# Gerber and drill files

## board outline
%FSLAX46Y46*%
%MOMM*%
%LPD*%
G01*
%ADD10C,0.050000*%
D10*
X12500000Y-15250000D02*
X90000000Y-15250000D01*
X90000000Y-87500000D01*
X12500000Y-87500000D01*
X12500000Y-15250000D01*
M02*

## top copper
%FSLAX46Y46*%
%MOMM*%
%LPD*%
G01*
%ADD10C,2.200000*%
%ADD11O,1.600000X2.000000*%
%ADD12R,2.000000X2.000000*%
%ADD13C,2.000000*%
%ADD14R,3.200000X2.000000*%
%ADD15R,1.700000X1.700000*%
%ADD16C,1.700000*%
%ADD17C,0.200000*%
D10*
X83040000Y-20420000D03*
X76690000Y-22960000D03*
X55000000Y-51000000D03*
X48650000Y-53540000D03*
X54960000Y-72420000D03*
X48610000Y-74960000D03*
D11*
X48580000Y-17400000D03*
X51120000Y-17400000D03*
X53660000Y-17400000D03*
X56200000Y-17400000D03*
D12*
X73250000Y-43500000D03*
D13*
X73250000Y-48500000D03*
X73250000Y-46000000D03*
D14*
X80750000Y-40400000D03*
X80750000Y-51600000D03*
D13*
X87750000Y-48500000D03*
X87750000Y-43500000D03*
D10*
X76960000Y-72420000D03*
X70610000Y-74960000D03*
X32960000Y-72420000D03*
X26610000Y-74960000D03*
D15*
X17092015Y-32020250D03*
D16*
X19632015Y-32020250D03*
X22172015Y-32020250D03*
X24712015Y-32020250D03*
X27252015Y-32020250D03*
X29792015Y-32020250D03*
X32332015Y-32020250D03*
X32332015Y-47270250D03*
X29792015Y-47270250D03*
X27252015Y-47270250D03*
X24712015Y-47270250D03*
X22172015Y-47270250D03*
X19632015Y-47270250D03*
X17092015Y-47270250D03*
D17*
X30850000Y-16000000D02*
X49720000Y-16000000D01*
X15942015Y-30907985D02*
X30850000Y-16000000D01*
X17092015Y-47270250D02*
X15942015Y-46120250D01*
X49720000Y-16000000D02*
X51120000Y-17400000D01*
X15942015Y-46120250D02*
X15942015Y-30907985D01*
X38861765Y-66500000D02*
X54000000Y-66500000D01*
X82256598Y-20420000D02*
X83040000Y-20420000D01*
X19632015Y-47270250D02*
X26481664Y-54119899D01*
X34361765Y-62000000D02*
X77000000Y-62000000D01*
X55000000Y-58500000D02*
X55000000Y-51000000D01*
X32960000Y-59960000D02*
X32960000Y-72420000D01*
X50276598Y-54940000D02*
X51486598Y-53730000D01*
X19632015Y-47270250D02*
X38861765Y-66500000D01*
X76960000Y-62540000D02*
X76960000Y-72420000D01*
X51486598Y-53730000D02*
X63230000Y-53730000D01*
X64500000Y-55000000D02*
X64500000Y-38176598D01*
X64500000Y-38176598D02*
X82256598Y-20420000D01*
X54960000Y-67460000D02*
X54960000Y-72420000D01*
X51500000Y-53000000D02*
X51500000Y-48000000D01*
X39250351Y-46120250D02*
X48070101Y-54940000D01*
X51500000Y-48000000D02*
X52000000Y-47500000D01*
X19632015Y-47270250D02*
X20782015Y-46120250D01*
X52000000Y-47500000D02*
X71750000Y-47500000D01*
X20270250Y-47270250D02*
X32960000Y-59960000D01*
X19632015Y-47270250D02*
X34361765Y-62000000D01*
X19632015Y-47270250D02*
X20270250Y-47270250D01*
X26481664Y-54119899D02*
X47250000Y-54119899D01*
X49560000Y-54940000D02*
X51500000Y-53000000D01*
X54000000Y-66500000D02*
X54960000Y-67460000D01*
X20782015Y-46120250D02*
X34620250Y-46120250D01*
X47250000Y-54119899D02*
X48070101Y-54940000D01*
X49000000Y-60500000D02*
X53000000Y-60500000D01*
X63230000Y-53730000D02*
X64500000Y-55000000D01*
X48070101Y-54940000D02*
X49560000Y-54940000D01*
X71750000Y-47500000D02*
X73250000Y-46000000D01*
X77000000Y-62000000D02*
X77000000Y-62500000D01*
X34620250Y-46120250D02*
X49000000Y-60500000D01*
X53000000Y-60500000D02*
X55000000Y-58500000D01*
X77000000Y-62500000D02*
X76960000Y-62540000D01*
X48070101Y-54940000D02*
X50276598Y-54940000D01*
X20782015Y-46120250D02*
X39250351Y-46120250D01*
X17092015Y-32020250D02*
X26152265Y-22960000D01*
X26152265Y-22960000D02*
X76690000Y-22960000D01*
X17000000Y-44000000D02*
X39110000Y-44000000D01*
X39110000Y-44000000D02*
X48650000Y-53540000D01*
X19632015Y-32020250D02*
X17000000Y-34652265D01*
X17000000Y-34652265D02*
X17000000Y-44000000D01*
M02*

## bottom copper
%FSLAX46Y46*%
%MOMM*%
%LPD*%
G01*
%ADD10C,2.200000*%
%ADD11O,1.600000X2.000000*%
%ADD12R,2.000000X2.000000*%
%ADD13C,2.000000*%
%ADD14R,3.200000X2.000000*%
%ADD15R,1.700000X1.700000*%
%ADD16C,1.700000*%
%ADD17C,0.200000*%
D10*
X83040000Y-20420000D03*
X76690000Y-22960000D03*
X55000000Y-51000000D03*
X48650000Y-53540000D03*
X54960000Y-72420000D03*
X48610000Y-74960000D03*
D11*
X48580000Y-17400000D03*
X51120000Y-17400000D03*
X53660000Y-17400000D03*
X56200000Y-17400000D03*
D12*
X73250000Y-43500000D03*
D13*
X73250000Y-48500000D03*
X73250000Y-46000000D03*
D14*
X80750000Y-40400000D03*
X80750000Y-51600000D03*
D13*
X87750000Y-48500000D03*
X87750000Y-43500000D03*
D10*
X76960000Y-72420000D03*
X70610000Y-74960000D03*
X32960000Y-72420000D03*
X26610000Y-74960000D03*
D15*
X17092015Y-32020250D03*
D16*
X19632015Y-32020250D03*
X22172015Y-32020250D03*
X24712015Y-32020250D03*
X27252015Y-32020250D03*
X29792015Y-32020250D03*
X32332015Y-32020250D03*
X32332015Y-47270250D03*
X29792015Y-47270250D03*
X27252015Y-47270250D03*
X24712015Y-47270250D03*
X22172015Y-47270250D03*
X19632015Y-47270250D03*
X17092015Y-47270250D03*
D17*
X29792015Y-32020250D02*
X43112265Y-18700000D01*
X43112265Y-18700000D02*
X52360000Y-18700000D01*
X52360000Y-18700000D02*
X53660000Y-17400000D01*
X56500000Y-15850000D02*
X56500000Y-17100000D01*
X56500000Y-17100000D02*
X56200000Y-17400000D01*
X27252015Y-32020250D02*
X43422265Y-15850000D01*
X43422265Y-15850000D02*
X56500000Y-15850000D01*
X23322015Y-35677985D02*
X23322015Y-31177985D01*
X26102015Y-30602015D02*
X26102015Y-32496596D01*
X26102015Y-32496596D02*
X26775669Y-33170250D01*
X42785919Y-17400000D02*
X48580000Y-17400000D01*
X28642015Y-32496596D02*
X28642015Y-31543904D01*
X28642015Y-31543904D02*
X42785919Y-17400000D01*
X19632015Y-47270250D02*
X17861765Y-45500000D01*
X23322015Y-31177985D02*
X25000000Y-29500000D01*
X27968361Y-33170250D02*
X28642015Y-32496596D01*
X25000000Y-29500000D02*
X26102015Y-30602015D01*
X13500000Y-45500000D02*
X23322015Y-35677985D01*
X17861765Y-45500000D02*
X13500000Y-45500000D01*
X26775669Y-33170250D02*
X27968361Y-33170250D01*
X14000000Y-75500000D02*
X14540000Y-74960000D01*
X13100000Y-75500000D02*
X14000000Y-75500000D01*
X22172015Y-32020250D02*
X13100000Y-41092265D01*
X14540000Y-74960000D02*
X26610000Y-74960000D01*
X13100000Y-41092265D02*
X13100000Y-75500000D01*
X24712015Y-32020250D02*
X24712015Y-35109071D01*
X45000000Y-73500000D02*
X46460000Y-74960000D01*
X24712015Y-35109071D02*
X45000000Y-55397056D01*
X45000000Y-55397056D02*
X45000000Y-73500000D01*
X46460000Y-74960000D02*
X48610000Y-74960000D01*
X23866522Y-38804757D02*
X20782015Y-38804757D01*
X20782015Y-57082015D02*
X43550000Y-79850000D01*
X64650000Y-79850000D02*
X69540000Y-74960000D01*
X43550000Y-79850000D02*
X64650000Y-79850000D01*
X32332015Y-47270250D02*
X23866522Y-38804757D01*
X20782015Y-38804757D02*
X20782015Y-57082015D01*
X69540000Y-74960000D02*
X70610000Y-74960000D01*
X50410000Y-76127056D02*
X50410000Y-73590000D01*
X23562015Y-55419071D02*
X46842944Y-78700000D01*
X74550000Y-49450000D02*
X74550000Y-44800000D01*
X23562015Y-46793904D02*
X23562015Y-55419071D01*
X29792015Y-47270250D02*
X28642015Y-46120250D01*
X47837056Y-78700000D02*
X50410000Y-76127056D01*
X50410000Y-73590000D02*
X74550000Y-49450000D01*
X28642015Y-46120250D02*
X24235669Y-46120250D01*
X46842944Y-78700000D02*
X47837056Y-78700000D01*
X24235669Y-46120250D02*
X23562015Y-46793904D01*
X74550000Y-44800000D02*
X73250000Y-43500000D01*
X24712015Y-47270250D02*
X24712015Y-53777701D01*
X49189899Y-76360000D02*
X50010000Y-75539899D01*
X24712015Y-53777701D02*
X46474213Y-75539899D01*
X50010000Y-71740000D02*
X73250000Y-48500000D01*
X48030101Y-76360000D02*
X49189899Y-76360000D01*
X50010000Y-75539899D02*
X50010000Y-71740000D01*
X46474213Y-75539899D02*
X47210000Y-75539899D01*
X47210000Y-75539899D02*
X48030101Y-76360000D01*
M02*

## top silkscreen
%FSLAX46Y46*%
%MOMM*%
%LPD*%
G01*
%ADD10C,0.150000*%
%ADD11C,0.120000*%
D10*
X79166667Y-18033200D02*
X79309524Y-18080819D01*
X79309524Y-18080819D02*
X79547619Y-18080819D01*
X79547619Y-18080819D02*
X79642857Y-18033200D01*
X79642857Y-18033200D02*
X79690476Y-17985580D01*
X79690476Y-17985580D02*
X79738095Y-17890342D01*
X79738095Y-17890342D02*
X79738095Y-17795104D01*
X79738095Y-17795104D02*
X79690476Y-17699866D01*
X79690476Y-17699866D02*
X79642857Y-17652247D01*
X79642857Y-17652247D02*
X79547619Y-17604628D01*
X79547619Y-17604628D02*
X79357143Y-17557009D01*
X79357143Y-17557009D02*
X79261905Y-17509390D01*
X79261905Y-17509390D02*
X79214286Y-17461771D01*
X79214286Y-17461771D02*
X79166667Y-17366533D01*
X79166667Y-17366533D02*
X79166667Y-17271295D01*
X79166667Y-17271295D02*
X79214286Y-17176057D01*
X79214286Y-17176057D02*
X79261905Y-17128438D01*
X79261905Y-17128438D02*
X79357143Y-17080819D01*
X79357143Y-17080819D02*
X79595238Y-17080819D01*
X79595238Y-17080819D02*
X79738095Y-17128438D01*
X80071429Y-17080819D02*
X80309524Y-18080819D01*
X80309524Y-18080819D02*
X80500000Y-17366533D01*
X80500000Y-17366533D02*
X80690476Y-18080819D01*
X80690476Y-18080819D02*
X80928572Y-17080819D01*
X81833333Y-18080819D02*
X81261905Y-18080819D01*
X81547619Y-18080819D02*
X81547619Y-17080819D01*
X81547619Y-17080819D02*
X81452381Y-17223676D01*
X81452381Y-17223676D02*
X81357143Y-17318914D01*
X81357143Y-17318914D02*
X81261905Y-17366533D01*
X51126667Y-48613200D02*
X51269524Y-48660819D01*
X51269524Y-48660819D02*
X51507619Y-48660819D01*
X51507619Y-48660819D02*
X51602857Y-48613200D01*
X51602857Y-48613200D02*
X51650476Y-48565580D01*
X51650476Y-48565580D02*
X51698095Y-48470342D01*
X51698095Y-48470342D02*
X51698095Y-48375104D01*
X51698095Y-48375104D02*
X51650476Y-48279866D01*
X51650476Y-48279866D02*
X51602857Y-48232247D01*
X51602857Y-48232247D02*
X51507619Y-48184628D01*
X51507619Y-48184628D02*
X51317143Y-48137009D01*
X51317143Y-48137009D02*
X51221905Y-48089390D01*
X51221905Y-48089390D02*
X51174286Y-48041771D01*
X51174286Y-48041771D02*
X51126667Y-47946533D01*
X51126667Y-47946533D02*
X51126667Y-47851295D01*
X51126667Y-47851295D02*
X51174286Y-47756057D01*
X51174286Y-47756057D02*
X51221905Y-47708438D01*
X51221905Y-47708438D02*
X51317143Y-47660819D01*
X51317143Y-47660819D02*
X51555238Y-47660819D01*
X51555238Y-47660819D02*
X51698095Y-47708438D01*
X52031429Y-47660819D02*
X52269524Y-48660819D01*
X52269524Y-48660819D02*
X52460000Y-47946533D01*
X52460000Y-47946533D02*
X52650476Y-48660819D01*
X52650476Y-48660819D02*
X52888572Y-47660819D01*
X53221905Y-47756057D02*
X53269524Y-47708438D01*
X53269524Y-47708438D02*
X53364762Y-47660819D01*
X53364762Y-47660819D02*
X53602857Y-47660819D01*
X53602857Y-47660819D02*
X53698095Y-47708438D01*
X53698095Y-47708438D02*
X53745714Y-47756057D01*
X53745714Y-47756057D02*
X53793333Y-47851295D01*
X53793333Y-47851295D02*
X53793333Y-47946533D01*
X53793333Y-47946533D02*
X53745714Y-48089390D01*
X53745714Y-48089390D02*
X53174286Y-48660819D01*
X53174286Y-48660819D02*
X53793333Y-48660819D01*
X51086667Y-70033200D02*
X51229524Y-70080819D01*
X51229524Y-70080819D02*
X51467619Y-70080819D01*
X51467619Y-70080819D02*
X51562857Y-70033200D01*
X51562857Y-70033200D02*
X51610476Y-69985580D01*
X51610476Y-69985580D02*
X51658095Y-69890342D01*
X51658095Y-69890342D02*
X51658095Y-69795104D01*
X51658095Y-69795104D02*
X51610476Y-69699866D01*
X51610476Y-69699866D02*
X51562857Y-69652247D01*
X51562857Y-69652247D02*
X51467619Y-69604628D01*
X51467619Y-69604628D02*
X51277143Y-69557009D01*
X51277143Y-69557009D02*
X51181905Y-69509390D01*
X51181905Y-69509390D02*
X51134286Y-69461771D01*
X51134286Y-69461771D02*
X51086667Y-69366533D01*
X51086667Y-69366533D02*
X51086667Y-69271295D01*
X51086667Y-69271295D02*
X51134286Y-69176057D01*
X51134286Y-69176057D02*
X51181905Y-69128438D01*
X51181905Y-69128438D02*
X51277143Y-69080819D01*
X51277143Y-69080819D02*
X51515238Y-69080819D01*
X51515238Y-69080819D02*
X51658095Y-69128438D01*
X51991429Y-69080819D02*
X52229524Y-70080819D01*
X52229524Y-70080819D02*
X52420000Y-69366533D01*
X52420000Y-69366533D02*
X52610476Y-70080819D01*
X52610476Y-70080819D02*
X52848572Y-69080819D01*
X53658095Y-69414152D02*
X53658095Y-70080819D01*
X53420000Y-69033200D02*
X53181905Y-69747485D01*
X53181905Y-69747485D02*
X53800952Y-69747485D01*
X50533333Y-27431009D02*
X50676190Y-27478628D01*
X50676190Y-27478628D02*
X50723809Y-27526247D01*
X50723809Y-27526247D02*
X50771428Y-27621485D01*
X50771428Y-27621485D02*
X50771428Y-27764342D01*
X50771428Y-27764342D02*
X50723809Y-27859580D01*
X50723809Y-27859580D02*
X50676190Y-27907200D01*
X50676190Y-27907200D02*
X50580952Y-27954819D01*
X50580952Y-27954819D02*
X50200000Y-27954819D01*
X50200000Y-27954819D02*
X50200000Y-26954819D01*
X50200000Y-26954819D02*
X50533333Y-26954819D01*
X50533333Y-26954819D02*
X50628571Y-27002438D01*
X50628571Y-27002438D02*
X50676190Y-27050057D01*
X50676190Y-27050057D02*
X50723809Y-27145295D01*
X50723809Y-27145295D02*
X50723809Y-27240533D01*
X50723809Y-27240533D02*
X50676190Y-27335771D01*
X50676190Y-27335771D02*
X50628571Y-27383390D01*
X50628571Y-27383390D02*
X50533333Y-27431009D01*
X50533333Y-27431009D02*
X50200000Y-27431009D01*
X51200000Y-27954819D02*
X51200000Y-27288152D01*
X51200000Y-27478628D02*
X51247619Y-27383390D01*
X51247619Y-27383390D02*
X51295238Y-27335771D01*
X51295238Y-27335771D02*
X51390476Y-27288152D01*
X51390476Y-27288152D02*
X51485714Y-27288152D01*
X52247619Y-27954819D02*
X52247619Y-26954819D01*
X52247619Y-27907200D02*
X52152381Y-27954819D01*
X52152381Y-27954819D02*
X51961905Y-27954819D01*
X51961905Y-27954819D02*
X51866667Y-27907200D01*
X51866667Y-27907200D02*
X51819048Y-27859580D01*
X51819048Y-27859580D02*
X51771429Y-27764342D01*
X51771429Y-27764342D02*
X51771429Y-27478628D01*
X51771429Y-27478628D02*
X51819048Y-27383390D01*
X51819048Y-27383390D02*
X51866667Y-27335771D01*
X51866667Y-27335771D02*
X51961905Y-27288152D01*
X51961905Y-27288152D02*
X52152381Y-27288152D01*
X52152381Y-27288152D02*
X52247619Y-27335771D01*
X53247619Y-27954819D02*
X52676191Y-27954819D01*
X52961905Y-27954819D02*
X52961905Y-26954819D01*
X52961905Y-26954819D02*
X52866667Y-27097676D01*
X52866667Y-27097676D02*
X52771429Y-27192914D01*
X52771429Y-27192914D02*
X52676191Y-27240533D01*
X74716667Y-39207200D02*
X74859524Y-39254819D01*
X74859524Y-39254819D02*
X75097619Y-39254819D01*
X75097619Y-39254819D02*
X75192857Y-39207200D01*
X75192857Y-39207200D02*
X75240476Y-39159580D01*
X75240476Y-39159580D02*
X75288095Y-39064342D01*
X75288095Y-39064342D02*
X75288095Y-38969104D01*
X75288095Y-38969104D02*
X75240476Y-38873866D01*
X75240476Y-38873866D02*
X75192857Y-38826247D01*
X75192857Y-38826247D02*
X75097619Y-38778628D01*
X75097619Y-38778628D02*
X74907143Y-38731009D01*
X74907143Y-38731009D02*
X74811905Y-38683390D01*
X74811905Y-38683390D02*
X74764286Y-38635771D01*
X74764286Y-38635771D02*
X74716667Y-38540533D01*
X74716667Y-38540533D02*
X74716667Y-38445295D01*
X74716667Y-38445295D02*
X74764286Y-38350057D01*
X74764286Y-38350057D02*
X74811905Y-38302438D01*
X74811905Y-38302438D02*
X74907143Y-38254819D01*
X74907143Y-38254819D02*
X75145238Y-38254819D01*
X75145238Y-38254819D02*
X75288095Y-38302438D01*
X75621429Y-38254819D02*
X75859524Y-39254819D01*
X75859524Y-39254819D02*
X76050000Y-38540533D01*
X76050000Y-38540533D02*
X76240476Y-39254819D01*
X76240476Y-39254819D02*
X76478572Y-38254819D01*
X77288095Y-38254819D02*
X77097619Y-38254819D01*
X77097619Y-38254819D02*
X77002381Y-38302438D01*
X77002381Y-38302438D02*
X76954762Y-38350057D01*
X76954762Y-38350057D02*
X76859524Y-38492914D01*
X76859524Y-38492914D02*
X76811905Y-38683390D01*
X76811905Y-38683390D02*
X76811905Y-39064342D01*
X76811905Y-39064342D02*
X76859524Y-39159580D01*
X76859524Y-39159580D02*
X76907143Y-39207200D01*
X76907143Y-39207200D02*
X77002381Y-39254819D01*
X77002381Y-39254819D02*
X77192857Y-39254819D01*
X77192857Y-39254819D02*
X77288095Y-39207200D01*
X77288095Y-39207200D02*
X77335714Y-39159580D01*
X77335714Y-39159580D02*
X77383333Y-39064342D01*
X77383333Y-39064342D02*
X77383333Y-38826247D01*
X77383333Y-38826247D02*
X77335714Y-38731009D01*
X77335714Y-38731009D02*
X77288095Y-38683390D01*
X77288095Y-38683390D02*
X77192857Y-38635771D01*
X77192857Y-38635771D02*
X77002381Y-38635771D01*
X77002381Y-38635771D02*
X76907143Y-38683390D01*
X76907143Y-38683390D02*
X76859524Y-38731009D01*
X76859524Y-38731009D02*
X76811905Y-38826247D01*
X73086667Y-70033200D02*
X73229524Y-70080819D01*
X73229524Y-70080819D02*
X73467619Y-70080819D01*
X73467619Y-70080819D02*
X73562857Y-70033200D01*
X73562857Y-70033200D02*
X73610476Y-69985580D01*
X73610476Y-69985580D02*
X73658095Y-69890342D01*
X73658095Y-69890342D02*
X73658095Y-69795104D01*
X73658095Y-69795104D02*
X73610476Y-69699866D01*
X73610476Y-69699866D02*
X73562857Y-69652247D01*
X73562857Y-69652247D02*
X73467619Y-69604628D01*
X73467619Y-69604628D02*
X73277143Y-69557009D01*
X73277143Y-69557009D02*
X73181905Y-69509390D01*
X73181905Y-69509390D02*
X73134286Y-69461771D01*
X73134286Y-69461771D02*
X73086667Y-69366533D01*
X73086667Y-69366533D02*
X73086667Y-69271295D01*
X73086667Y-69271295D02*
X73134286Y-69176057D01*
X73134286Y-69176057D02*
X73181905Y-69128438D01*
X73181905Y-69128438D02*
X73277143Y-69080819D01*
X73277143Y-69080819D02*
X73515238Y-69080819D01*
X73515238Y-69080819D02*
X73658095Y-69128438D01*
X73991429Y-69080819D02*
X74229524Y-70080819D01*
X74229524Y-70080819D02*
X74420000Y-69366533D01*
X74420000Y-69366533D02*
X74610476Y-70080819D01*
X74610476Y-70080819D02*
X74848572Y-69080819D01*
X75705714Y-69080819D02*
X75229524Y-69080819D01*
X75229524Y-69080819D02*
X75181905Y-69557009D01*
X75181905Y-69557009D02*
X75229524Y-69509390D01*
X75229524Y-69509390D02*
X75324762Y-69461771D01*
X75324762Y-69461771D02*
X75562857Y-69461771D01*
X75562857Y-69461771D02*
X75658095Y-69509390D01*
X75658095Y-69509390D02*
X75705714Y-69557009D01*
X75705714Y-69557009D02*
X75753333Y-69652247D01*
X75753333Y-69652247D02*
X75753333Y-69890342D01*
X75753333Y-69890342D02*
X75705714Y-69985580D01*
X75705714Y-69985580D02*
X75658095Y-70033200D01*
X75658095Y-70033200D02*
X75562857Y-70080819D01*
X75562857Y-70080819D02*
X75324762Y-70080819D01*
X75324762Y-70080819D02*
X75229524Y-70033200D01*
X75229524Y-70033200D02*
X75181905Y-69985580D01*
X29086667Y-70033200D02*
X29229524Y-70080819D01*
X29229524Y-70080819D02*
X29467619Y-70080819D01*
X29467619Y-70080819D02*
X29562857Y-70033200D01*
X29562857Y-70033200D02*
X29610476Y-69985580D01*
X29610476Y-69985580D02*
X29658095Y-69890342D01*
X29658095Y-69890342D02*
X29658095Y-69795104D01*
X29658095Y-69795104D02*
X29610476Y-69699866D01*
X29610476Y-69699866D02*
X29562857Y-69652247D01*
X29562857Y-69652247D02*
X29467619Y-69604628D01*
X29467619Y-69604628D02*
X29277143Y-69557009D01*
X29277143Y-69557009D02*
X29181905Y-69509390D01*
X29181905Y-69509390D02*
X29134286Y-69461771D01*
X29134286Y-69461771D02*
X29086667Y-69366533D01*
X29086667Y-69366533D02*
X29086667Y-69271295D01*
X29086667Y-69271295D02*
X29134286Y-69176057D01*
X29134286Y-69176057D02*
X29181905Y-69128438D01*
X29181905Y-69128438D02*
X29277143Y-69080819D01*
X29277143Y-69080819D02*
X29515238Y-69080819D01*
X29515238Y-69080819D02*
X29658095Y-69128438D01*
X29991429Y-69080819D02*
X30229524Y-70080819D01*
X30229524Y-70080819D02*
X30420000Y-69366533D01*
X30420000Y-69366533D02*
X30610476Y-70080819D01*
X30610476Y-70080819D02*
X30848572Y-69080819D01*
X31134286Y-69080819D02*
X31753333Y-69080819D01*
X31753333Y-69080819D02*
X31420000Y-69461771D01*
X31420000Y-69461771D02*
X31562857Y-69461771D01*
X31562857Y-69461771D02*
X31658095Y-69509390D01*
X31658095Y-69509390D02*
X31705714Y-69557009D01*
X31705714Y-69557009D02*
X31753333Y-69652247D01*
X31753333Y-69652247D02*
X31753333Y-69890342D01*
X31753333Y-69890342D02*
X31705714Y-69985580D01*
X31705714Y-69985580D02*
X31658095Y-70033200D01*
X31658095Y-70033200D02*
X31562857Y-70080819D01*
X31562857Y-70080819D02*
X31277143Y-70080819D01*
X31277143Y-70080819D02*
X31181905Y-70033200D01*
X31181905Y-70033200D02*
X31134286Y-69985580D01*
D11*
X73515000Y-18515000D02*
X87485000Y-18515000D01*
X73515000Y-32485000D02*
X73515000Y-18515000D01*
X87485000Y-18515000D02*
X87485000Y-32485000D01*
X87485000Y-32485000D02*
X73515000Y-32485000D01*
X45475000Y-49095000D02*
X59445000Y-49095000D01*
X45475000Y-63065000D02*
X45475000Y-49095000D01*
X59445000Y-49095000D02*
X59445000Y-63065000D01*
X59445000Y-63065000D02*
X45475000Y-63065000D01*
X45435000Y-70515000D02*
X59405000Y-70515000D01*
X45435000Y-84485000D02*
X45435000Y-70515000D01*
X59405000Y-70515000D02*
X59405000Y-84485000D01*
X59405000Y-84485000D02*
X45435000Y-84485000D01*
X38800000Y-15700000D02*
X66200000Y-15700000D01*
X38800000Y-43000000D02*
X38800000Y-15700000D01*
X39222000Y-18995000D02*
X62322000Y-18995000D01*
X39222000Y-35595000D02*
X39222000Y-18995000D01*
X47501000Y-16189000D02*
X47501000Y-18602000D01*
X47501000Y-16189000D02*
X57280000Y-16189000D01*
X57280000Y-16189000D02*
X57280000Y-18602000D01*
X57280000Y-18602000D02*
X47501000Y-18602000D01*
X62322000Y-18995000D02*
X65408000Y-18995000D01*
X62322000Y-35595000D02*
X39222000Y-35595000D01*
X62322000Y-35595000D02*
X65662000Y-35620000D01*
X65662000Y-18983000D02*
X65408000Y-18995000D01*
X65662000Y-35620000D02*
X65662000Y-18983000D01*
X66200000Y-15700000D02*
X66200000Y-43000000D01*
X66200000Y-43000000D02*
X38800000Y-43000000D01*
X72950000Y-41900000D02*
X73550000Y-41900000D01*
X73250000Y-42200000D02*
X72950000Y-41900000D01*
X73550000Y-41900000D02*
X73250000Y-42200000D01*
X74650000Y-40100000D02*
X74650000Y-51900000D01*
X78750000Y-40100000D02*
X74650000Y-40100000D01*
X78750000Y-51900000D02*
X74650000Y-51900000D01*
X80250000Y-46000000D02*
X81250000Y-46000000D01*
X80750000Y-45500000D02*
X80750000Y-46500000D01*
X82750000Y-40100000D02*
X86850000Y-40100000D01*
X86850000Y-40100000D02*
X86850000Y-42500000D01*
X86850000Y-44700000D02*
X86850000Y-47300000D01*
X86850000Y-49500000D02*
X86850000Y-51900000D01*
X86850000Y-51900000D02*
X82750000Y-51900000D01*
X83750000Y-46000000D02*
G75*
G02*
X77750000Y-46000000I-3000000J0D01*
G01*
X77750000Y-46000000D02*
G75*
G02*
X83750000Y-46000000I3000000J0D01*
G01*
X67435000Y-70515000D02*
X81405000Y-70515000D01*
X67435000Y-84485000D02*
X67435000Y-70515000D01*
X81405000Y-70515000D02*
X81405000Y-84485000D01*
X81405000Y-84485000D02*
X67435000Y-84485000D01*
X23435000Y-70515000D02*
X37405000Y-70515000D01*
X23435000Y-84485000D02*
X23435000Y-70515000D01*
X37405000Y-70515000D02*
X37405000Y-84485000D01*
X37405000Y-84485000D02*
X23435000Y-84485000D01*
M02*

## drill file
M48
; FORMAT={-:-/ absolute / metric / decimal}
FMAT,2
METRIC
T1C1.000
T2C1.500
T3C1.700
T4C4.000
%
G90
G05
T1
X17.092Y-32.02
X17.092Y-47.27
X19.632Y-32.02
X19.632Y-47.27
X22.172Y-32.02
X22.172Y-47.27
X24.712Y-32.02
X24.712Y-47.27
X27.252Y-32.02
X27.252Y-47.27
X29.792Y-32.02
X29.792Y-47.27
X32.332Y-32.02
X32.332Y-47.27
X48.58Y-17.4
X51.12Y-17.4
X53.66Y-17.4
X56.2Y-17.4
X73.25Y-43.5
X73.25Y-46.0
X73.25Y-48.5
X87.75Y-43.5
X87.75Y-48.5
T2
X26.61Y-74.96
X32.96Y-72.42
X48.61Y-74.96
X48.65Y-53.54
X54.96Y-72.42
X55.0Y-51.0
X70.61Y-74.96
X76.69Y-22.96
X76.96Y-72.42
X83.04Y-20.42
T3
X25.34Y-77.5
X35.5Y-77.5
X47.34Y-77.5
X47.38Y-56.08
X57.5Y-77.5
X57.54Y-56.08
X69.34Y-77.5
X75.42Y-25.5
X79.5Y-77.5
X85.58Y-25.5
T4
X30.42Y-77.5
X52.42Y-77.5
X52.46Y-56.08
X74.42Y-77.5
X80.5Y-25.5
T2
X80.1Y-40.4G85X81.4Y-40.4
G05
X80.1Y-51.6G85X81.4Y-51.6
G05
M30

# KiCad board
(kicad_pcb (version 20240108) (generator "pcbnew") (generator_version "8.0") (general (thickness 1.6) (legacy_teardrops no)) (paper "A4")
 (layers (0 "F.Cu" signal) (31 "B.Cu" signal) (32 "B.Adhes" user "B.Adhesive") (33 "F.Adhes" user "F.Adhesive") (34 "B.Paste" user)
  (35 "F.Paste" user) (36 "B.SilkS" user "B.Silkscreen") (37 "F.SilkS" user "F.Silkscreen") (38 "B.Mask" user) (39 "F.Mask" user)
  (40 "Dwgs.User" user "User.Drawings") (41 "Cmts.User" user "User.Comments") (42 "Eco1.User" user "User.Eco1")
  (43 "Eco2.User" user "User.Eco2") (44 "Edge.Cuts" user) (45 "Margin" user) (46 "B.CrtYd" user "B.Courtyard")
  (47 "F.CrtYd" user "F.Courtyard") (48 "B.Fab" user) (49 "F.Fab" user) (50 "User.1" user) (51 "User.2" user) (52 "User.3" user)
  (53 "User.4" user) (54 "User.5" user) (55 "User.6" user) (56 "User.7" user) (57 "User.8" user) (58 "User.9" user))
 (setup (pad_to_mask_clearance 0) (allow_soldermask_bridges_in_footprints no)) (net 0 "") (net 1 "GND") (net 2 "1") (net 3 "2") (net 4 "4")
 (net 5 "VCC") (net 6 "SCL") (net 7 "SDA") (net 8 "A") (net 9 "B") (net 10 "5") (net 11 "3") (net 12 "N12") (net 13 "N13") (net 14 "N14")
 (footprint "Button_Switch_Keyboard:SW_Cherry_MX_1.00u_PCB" (layer "F.Cu") (at 83.04 20.42)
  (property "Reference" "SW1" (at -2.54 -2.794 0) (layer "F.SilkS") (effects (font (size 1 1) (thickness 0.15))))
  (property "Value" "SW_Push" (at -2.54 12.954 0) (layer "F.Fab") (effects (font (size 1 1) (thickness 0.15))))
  (fp_line (start -9.525 -1.905) (end 4.445 -1.905) (stroke (width 0.12) (type solid)) (layer "F.SilkS"))
  (fp_line (start -9.525 12.065) (end -9.525 -1.905) (stroke (width 0.12) (type solid)) (layer "F.SilkS"))
  (fp_line (start 4.445 -1.905) (end 4.445 12.065) (stroke (width 0.12) (type solid)) (layer "F.SilkS"))
  (fp_line (start 4.445 12.065) (end -9.525 12.065) (stroke (width 0.12) (type solid)) (layer "F.SilkS"))
  (pad "" np_thru_hole circle (at -7.62 5.08) (size 1.7 1.7) (drill 1.7) (layers "*.Cu" "*.Mask"))
  (pad "" np_thru_hole circle (at -2.54 5.08) (size 4 4) (drill 4) (layers "*.Cu" "*.Mask"))
  (pad "" np_thru_hole circle (at 2.54 5.08) (size 1.7 1.7) (drill 1.7) (layers "*.Cu" "*.Mask"))
  (pad "1" thru_hole circle (at 0 0) (size 2.2 2.2) (drill 1.5) (layers "*.Cu" "*.Mask") (remove_unused_layers no) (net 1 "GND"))
  (pad "2" thru_hole circle (at -6.35 2.54) (size 2.2 2.2) (drill 1.5) (layers "*.Cu" "*.Mask") (remove_unused_layers no) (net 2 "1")))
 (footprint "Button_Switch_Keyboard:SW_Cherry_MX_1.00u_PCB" (layer "F.Cu") (at 55 51)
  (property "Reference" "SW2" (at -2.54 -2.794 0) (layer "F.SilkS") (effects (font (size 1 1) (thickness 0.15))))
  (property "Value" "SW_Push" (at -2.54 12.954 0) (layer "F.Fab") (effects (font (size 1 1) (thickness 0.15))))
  (fp_line (start -9.525 -1.905) (end 4.445 -1.905) (stroke (width 0.12) (type solid)) (layer "F.SilkS"))
  (fp_line (start -9.525 12.065) (end -9.525 -1.905) (stroke (width 0.12) (type solid)) (layer "F.SilkS"))
  (fp_line (start 4.445 -1.905) (end 4.445 12.065) (stroke (width 0.12) (type solid)) (layer "F.SilkS"))
  (fp_line (start 4.445 12.065) (end -9.525 12.065) (stroke (width 0.12) (type solid)) (layer "F.SilkS"))
  (pad "" np_thru_hole circle (at -7.62 5.08) (size 1.7 1.7) (drill 1.7) (layers "*.Cu" "*.Mask"))
  (pad "" np_thru_hole circle (at -2.54 5.08) (size 4 4) (drill 4) (layers "*.Cu" "*.Mask"))
  (pad "" np_thru_hole circle (at 2.54 5.08) (size 1.7 1.7) (drill 1.7) (layers "*.Cu" "*.Mask"))
  (pad "1" thru_hole circle (at 0 0) (size 2.2 2.2) (drill 1.5) (layers "*.Cu" "*.Mask") (remove_unused_layers no) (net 1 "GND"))
  (pad "2" thru_hole circle (at -6.35 2.54) (size 2.2 2.2) (drill 1.5) (layers "*.Cu" "*.Mask") (remove_unused_layers no) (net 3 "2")))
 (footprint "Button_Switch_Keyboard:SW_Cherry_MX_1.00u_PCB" (layer "F.Cu") (at 54.96 72.42)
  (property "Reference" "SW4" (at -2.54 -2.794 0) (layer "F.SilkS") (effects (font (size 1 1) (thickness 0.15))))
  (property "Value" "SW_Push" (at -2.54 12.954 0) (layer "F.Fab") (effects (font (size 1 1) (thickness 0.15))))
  (fp_line (start -9.525 -1.905) (end 4.445 -1.905) (stroke (width 0.12) (type solid)) (layer "F.SilkS"))
  (fp_line (start -9.525 12.065) (end -9.525 -1.905) (stroke (width 0.12) (type solid)) (layer "F.SilkS"))
  (fp_line (start 4.445 -1.905) (end 4.445 12.065) (stroke (width 0.12) (type solid)) (layer "F.SilkS"))
  (fp_line (start 4.445 12.065) (end -9.525 12.065) (stroke (width 0.12) (type solid)) (layer "F.SilkS"))
  (pad "" np_thru_hole circle (at -7.62 5.08) (size 1.7 1.7) (drill 1.7) (layers "*.Cu" "*.Mask"))
  (pad "" np_thru_hole circle (at -2.54 5.08) (size 4 4) (drill 4) (layers "*.Cu" "*.Mask"))
  (pad "" np_thru_hole circle (at 2.54 5.08) (size 1.7 1.7) (drill 1.7) (layers "*.Cu" "*.Mask"))
  (pad "1" thru_hole circle (at 0 0) (size 2.2 2.2) (drill 1.5) (layers "*.Cu" "*.Mask") (remove_unused_layers no) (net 1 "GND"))
  (pad "2" thru_hole circle (at -6.35 2.54) (size 2.2 2.2) (drill 1.5) (layers "*.Cu" "*.Mask") (remove_unused_layers no) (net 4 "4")))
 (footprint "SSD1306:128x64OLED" (layer "F.Cu") (at 52.2 28)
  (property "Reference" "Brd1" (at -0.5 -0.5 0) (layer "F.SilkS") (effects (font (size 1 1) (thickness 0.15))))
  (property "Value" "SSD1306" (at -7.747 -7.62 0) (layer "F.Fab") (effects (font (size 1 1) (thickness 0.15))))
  (fp_line (start -13.4 -12.3) (end 14 -12.3) (stroke (width 0.12) (type solid)) (layer "F.SilkS"))
  (fp_line (start -13.4 15) (end -13.4 -12.3) (stroke (width 0.12) (type solid)) (layer "F.SilkS"))
  (fp_line (start -12.978 -9.005) (end 10.122 -9.005) (stroke (width 0.12) (type solid)) (layer "F.SilkS"))
  (fp_line (start -12.978 7.595) (end -12.978 -9.005) (stroke (width 0.12) (type solid)) (layer "F.SilkS"))
  (fp_line (start -4.699 -11.811) (end -4.699 -9.398) (stroke (width 0.12) (type solid)) (layer "F.SilkS"))
  (fp_line (start -4.699 -11.811) (end 5.08 -11.811) (stroke (width 0.12) (type solid)) (layer "F.SilkS"))
  (fp_line (start 5.08 -11.811) (end 5.08 -9.398) (stroke (width 0.12) (type solid)) (layer "F.SilkS"))
  (fp_line (start 5.08 -9.398) (end -4.699 -9.398) (stroke (width 0.12) (type solid)) (layer "F.SilkS"))
  (fp_line (start 10.122 -9.005) (end 13.208 -9.005) (stroke (width 0.12) (type solid)) (layer "F.SilkS"))
  (fp_line (start 10.122 7.595) (end -12.978 7.595) (stroke (width 0.12) (type solid)) (layer "F.SilkS"))
  (fp_line (start 10.122 7.595) (end 13.462 7.62) (stroke (width 0.12) (type solid)) (layer "F.SilkS"))
  (fp_line (start 13.462 -9.017) (end 13.208 -9.005) (stroke (width 0.12) (type solid)) (layer "F.SilkS"))
  (fp_line (start 13.462 7.62) (end 13.462 -9.017) (stroke (width 0.12) (type solid)) (layer "F.SilkS"))
  (fp_line (start 14 -12.3) (end 14 15) (stroke (width 0.12) (type solid)) (layer "F.SilkS"))
  (fp_line (start 14 15) (end -13.4 15) (stroke (width 0.12) (type solid)) (layer "F.SilkS"))
  (pad "1" thru_hole oval (at -3.62 -10.6 90) (size 2 1.6) (drill 1) (layers "*.Cu" "*.Mask") (remove_unused_layers no) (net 1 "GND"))
  (pad "2" thru_hole oval (at -1.08 -10.6 90) (size 2 1.6) (drill 1) (layers "*.Cu" "*.Mask") (remove_unused_layers no) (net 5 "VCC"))
  (pad "3" thru_hole oval (at 1.46 -10.6 90) (size 2 1.6) (drill 1) (layers "*.Cu" "*.Mask") (remove_unused_layers no) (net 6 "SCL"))
  (pad "4" thru_hole oval (at 4 -10.6 90) (size 2 1.6) (drill 1) (layers "*.Cu" "*.Mask") (remove_unused_layers no) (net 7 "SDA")))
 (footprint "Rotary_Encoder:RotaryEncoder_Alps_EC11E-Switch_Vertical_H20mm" (layer "F.Cu") (at 73.25 43.5)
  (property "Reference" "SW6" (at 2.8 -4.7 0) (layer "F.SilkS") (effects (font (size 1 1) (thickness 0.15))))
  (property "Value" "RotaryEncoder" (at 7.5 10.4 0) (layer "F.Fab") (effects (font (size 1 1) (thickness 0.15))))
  (fp_line (start -0.3 -1.6) (end 0.3 -1.6) (stroke (width 0.12) (type solid)) (layer "F.SilkS"))
  (fp_line (start 0 -1.3) (end -0.3 -1.6) (stroke (width 0.12) (type solid)) (layer "F.SilkS"))
  (fp_line (start 0.3 -1.6) (end 0 -1.3) (stroke (width 0.12) (type solid)) (layer "F.SilkS"))
  (fp_line (start 1.4 -3.4) (end 1.4 8.4) (stroke (width 0.12) (type solid)) (layer "F.SilkS"))
  (fp_line (start 5.5 -3.4) (end 1.4 -3.4) (stroke (width 0.12) (type solid)) (layer "F.SilkS"))
  (fp_line (start 5.5 8.4) (end 1.4 8.4) (stroke (width 0.12) (type solid)) (layer "F.SilkS"))
  (fp_line (start 7 2.5) (end 8 2.5) (stroke (width 0.12) (type solid)) (layer "F.SilkS"))
  (fp_line (start 7.5 2) (end 7.5 3) (stroke (width 0.12) (type solid)) (layer "F.SilkS"))
  (fp_line (start 9.5 -3.4) (end 13.6 -3.4) (stroke (width 0.12) (type solid)) (layer "F.SilkS"))
  (fp_line (start 13.6 -3.4) (end 13.6 -1) (stroke (width 0.12) (type solid)) (layer "F.SilkS"))
  (fp_line (start 13.6 1.2) (end 13.6 3.8) (stroke (width 0.12) (type solid)) (layer "F.SilkS"))
  (fp_line (start 13.6 6) (end 13.6 8.4) (stroke (width 0.12) (type solid)) (layer "F.SilkS"))
  (fp_line (start 13.6 8.4) (end 9.5 8.4) (stroke (width 0.12) (type solid)) (layer "F.SilkS"))
  (fp_circle (center 7.5 2.5) (end 10.5 2.5) (stroke (width 0.12) (type solid)) (fill none) (layer "F.SilkS"))
  (pad "A" thru_hole rect (at 0 0) (size 2 2) (drill 1) (layers "*.Cu" "*.Mask") (remove_unused_layers no) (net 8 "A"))
  (pad "B" thru_hole circle (at 0 5) (size 2 2) (drill 1) (layers "*.Cu" "*.Mask") (remove_unused_layers no) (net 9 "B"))
  (pad "C" thru_hole circle (at 0 2.5) (size 2 2) (drill 1) (layers "*.Cu" "*.Mask") (remove_unused_layers no) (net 1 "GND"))
  (pad "MP" thru_hole rect (at 7.5 -3.1) (size 3.2 2) (drill oval 2.8 1.5) (layers "*.Cu" "*.Mask") (remove_unused_layers no))
  (pad "MP" thru_hole rect (at 7.5 8.1) (size 3.2 2) (drill oval 2.8 1.5) (layers "*.Cu" "*.Mask") (remove_unused_layers no))
  (pad "S1" thru_hole circle (at 14.5 5) (size 2 2) (drill 1) (layers "*.Cu" "*.Mask") (remove_unused_layers no))
  (pad "S2" thru_hole circle (at 14.5 0) (size 2 2) (drill 1) (layers "*.Cu" "*.Mask") (remove_unused_layers no)))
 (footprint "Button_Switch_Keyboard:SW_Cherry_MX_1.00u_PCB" (layer "F.Cu") (at 76.96 72.42)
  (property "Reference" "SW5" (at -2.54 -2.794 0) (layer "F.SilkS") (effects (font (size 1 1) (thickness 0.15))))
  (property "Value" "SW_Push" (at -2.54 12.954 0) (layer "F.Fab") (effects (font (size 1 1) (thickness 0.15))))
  (fp_line (start -9.525 -1.905) (end 4.445 -1.905) (stroke (width 0.12) (type solid)) (layer "F.SilkS"))
  (fp_line (start -9.525 12.065) (end -9.525 -1.905) (stroke (width 0.12) (type solid)) (layer "F.SilkS"))
  (fp_line (start 4.445 -1.905) (end 4.445 12.065) (stroke (width 0.12) (type solid)) (layer "F.SilkS"))
  (fp_line (start 4.445 12.065) (end -9.525 12.065) (stroke (width 0.12) (type solid)) (layer "F.SilkS"))
  (pad "" np_thru_hole circle (at -7.62 5.08) (size 1.7 1.7) (drill 1.7) (layers "*.Cu" "*.Mask"))
  (pad "" np_thru_hole circle (at -2.54 5.08) (size 4 4) (drill 4) (layers "*.Cu" "*.Mask"))
  (pad "" np_thru_hole circle (at 2.54 5.08) (size 1.7 1.7) (drill 1.7) (layers "*.Cu" "*.Mask"))
  (pad "1" thru_hole circle (at 0 0) (size 2.2 2.2) (drill 1.5) (layers "*.Cu" "*.Mask") (remove_unused_layers no) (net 1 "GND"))
  (pad "2" thru_hole circle (at -6.35 2.54) (size 2.2 2.2) (drill 1.5) (layers "*.Cu" "*.Mask") (remove_unused_layers no) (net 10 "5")))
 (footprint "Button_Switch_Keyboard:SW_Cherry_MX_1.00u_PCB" (layer "F.Cu") (at 32.96 72.42)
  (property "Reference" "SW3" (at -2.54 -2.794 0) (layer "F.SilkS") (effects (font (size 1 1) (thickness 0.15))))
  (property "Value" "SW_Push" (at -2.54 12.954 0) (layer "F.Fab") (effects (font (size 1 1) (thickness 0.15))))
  (fp_line (start -9.525 -1.905) (end 4.445 -1.905) (stroke (width 0.12) (type solid)) (layer "F.SilkS"))
  (fp_line (start -9.525 12.065) (end -9.525 -1.905) (stroke (width 0.12) (type solid)) (layer "F.SilkS"))
  (fp_line (start 4.445 -1.905) (end 4.445 12.065) (stroke (width 0.12) (type solid)) (layer "F.SilkS"))
  (fp_line (start 4.445 12.065) (end -9.525 12.065) (stroke (width 0.12) (type solid)) (layer "F.SilkS"))
  (pad "" np_thru_hole circle (at -7.62 5.08) (size 1.7 1.7) (drill 1.7) (layers "*.Cu" "*.Mask"))
  (pad "" np_thru_hole circle (at -2.54 5.08) (size 4 4) (drill 4) (layers "*.Cu" "*.Mask"))
  (pad "" np_thru_hole circle (at 2.54 5.08) (size 1.7 1.7) (drill 1.7) (layers "*.Cu" "*.Mask"))
  (pad "1" thru_hole circle (at 0 0) (size 2.2 2.2) (drill 1.5) (layers "*.Cu" "*.Mask") (remove_unused_layers no) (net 1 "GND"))
  (pad "2" thru_hole circle (at -6.35 2.54) (size 2.2 2.2) (drill 1.5) (layers "*.Cu" "*.Mask") (remove_unused_layers no) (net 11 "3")))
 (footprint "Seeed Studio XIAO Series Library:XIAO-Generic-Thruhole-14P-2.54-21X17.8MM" (layer "B.Cu") (at 24.712015 39.64525 -90)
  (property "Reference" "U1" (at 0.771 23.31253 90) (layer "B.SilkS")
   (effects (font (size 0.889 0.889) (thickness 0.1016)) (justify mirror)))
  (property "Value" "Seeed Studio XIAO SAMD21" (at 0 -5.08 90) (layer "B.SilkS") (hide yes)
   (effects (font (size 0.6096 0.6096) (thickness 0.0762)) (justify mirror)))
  (pad "1" thru_hole rect (at -7.625 7.62 270) (size 1.7 1.7) (drill 1) (layers "*.Cu" "*.Mask") (remove_unused_layers no) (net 2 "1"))
  (pad "2" thru_hole circle (at -7.625 5.08 270) (size 1.7 1.7) (drill 1) (layers "*.Cu" "*.Mask") (remove_unused_layers no) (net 3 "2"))
  (pad "3" thru_hole circle (at -7.625 2.54 270) (size 1.7 1.7) (drill 1) (layers "*.Cu" "*.Mask") (remove_unused_layers no) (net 11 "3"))
  (pad "4" thru_hole circle (at -7.625 0 270) (size 1.7 1.7) (drill 1) (layers "*.Cu" "*.Mask") (remove_unused_layers no) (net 4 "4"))
  (pad "5" thru_hole circle (at -7.625 -2.54 270) (size 1.7 1.7) (drill 1) (layers "*.Cu" "*.Mask") (remove_unused_layers no) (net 7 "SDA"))
  (pad "6" thru_hole circle (at -7.625 -5.08 90) (size 1.7 1.7) (drill 1) (layers "*.Cu" "*.Mask") (remove_unused_layers no) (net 6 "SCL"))
  (pad "7" thru_hole circle (at -7.625 -7.62 270) (size 1.7 1.7) (drill 1) (layers "*.Cu" "*.Mask") (remove_unused_layers no) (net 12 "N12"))
  (pad "8" thru_hole circle (at 7.625 -7.62 270) (size 1.7 1.7) (drill 1) (layers "*.Cu" "*.Mask") (remove_unused_layers no) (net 10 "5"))
  (pad "9" thru_hole circle (at 7.625 -5.08 270) (size 1.7 1.7) (drill 1) (layers "*.Cu" "*.Mask") (remove_unused_layers no) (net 8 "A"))
  (pad "10" thru_hole circle (at 7.625 -2.54 270) (size 1.7 1.7) (drill 1) (layers "*.Cu" "*.Mask") (remove_unused_layers no) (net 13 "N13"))
  (pad "11" thru_hole circle (at 7.625 0 270) (size 1.7 1.7) (drill 1) (layers "*.Cu" "*.Mask") (remove_unused_layers no) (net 9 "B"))
  (pad "12" thru_hole circle (at 7.625 2.54 270) (size 1.7 1.7) (drill 1) (layers "*.Cu" "*.Mask") (remove_unused_layers no) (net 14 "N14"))
  (pad "13" thru_hole circle (at 7.625 5.08 270) (size 1.7 1.7) (drill 1) (layers "*.Cu" "*.Mask") (remove_unused_layers no) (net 1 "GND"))
  (pad "14" thru_hole circle (at 7.625 7.62 270) (size 1.7 1.7) (drill 1) (layers "*.Cu" "*.Mask") (remove_unused_layers no) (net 5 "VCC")))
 (gr_rect (start 12.5 15.25) (end 90 87.5) (stroke (width 0.05) (type default)) (fill none) (layer "Edge.Cuts"))
 (segment (start 30.85 16) (end 49.72 16) (width 0.2) (layer "F.Cu") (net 5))
 (segment (start 15.942015 30.907985) (end 30.85 16) (width 0.2) (layer "F.Cu") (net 5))
 (segment (start 17.092015 47.27025) (end 15.942015 46.12025) (width 0.2) (layer "F.Cu") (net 5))
 (segment (start 49.72 16) (end 51.12 17.4) (width 0.2) (layer "F.Cu") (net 5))
 (segment (start 15.942015 46.12025) (end 15.942015 30.907985) (width 0.2) (layer "F.Cu") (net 5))
 (segment (start 29.792015 32.02025) (end 43.112265 18.7) (width 0.2) (layer "B.Cu") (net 6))
 (segment (start 43.112265 18.7) (end 52.36 18.7) (width 0.2) (layer "B.Cu") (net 6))
 (segment (start 52.36 18.7) (end 53.66 17.4) (width 0.2) (layer "B.Cu") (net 6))
 (segment (start 56.5 15.85) (end 56.5 17.1) (width 0.2) (layer "B.Cu") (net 7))
 (segment (start 56.5 17.1) (end 56.2 17.4) (width 0.2) (layer "B.Cu") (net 7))
 (segment (start 27.252015 32.02025) (end 43.422265 15.85) (width 0.2) (layer "B.Cu") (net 7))
 (segment (start 43.422265 15.85) (end 56.5 15.85) (width 0.2) (layer "B.Cu") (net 7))
 (segment (start 38.861765 66.5) (end 54 66.5) (width 0.2) (layer "F.Cu") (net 1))
 (segment (start 82.256598 20.42) (end 83.04 20.42) (width 0.2) (layer "F.Cu") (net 1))
 (segment (start 19.632015 47.27025) (end 26.481664 54.119899) (width 0.2) (layer "F.Cu") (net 1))
 (segment (start 34.361765 62) (end 77 62) (width 0.2) (layer "F.Cu") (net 1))
 (segment (start 55 58.5) (end 55 51) (width 0.2) (layer "F.Cu") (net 1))
 (segment (start 32.96 59.96) (end 32.96 72.42) (width 0.2) (layer "F.Cu") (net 1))
 (segment (start 50.276598 54.94) (end 51.486598 53.73) (width 0.2) (layer "F.Cu") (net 1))
 (segment (start 19.632015 47.27025) (end 38.861765 66.5) (width 0.2) (layer "F.Cu") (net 1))
 (segment (start 76.96 62.54) (end 76.96 72.42) (width 0.2) (layer "F.Cu") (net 1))
 (segment (start 51.486598 53.73) (end 63.23 53.73) (width 0.2) (layer "F.Cu") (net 1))
 (segment (start 64.5 55) (end 64.5 38.176598) (width 0.2) (layer "F.Cu") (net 1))
 (segment (start 64.5 38.176598) (end 82.256598 20.42) (width 0.2) (layer "F.Cu") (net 1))
 (segment (start 54.96 67.46) (end 54.96 72.42) (width 0.2) (layer "F.Cu") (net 1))
 (segment (start 51.5 53) (end 51.5 48) (width 0.2) (layer "F.Cu") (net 1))
 (segment (start 39.250351 46.12025) (end 48.070101 54.94) (width 0.2) (layer "F.Cu") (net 1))
 (segment (start 51.5 48) (end 52 47.5) (width 0.2) (layer "F.Cu") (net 1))
 (segment (start 19.632015 47.27025) (end 20.782015 46.12025) (width 0.2) (layer "F.Cu") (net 1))
 (segment (start 52 47.5) (end 71.75 47.5) (width 0.2) (layer "F.Cu") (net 1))
 (segment (start 20.27025 47.27025) (end 32.96 59.96) (width 0.2) (layer "F.Cu") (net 1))
 (segment (start 19.632015 47.27025) (end 34.361765 62) (width 0.2) (layer "F.Cu") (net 1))
 (segment (start 19.632015 47.27025) (end 20.27025 47.27025) (width 0.2) (layer "F.Cu") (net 1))
 (segment (start 26.481664 54.119899) (end 47.25 54.119899) (width 0.2) (layer "F.Cu") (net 1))
 (segment (start 49.56 54.94) (end 51.5 53) (width 0.2) (layer "F.Cu") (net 1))
 (segment (start 54 66.5) (end 54.96 67.46) (width 0.2) (layer "F.Cu") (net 1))
 (segment (start 20.782015 46.12025) (end 34.62025 46.12025) (width 0.2) (layer "F.Cu") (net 1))
 (segment (start 47.25 54.119899) (end 48.070101 54.94) (width 0.2) (layer "F.Cu") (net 1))
 (segment (start 49 60.5) (end 53 60.5) (width 0.2) (layer "F.Cu") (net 1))
 (segment (start 63.23 53.73) (end 64.5 55) (width 0.2) (layer "F.Cu") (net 1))
 (segment (start 48.070101 54.94) (end 49.56 54.94) (width 0.2) (layer "F.Cu") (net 1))
 (segment (start 71.75 47.5) (end 73.25 46) (width 0.2) (layer "F.Cu") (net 1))
 (segment (start 77 62) (end 77 62.5) (width 0.2) (layer "F.Cu") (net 1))
 (segment (start 34.62025 46.12025) (end 49 60.5) (width 0.2) (layer "F.Cu") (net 1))
 (segment (start 53 60.5) (end 55 58.5) (width 0.2) (layer "F.Cu") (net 1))
 (segment (start 77 62.5) (end 76.96 62.54) (width 0.2) (layer "F.Cu") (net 1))
 (segment (start 48.070101 54.94) (end 50.276598 54.94) (width 0.2) (layer "F.Cu") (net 1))
 (segment (start 20.782015 46.12025) (end 39.250351 46.12025) (width 0.2) (layer "F.Cu") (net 1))
 (segment (start 23.322015 35.677985) (end 23.322015 31.177985) (width 0.2) (layer "B.Cu") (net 1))
 (segment (start 26.102015 30.602015) (end 26.102015 32.496596) (width 0.2) (layer "B.Cu") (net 1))
 (segment (start 26.102015 32.496596) (end 26.775669 33.17025) (width 0.2) (layer "B.Cu") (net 1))
 (segment (start 42.785919 17.4) (end 48.58 17.4) (width 0.2) (layer "B.Cu") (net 1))
 (segment (start 28.642015 32.496596) (end 28.642015 31.543904) (width 0.2) (layer "B.Cu") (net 1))
 (segment (start 28.642015 31.543904) (end 42.785919 17.4) (width 0.2) (layer "B.Cu") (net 1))
 (segment (start 19.632015 47.27025) (end 17.861765 45.5) (width 0.2) (layer "B.Cu") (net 1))
 (segment (start 23.322015 31.177985) (end 25 29.5) (width 0.2) (layer "B.Cu") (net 1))
 (segment (start 27.968361 33.17025) (end 28.642015 32.496596) (width 0.2) (layer "B.Cu") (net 1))
 (segment (start 25 29.5) (end 26.102015 30.602015) (width 0.2) (layer "B.Cu") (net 1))
 (segment (start 13.5 45.5) (end 23.322015 35.677985) (width 0.2) (layer "B.Cu") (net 1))
 (segment (start 17.861765 45.5) (end 13.5 45.5) (width 0.2) (layer "B.Cu") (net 1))
 (segment (start 26.775669 33.17025) (end 27.968361 33.17025) (width 0.2) (layer "B.Cu") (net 1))
 (segment (start 17.092015 32.02025) (end 26.152265 22.96) (width 0.2) (layer "F.Cu") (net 2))
 (segment (start 26.152265 22.96) (end 76.69 22.96) (width 0.2) (layer "F.Cu") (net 2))
 (segment (start 17 44) (end 39.11 44) (width 0.2) (layer "F.Cu") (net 3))
 (segment (start 39.11 44) (end 48.65 53.54) (width 0.2) (layer "F.Cu") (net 3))
 (segment (start 19.632015 32.02025) (end 17 34.652265) (width 0.2) (layer "F.Cu") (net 3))
 (segment (start 17 34.652265) (end 17 44) (width 0.2) (layer "F.Cu") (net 3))
 (segment (start 14 75.5) (end 14.54 74.96) (width 0.2) (layer "B.Cu") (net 11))
 (segment (start 13.1 75.5) (end 14 75.5) (width 0.2) (layer "B.Cu") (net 11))
 (segment (start 22.172015 32.02025) (end 13.1 41.092265) (width 0.2) (layer "B.Cu") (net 11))
 (segment (start 14.54 74.96) (end 26.61 74.96) (width 0.2) (layer "B.Cu") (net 11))
 (segment (start 13.1 41.092265) (end 13.1 75.5) (width 0.2) (layer "B.Cu") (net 11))
 (segment (start 24.712015 32.02025) (end 24.712015 35.109071) (width 0.2) (layer "B.Cu") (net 4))
 (segment (start 45 73.5) (end 46.46 74.96) (width 0.2) (layer "B.Cu") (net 4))
 (segment (start 24.712015 35.109071) (end 45 55.397056) (width 0.2) (layer "B.Cu") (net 4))
 (segment (start 45 55.397056) (end 45 73.5) (width 0.2) (layer "B.Cu") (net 4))
 (segment (start 46.46 74.96) (end 48.61 74.96) (width 0.2) (layer "B.Cu") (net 4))
 (segment (start 23.866522 38.804757) (end 20.782015 38.804757) (width 0.2) (layer "B.Cu") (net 10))
 (segment (start 20.782015 57.082015) (end 43.55 79.85) (width 0.2) (layer "B.Cu") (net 10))
 (segment (start 64.65 79.85) (end 69.54 74.96) (width 0.2) (layer "B.Cu") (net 10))
 (segment (start 43.55 79.85) (end 64.65 79.85) (width 0.2) (layer "B.Cu") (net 10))
 (segment (start 32.332015 47.27025) (end 23.866522 38.804757) (width 0.2) (layer "B.Cu") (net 10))
 (segment (start 20.782015 38.804757) (end 20.782015 57.082015) (width 0.2) (layer "B.Cu") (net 10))
 (segment (start 69.54 74.96) (end 70.61 74.96) (width 0.2) (layer "B.Cu") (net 10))
 (segment (start 50.41 76.127056) (end 50.41 73.59) (width 0.2) (layer "B.Cu") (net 8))
 (segment (start 23.562015 55.419071) (end 46.842944 78.7) (width 0.2) (layer "B.Cu") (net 8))
 (segment (start 74.55 49.45) (end 74.55 44.8) (width 0.2) (layer "B.Cu") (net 8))
 (segment (start 23.562015 46.793904) (end 23.562015 55.419071) (width 0.2) (layer "B.Cu") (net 8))
 (segment (start 29.792015 47.27025) (end 28.642015 46.12025) (width 0.2) (layer "B.Cu") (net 8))
 (segment (start 47.837056 78.7) (end 50.41 76.127056) (width 0.2) (layer "B.Cu") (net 8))
 (segment (start 50.41 73.59) (end 74.55 49.45) (width 0.2) (layer "B.Cu") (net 8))
 (segment (start 28.642015 46.12025) (end 24.235669 46.12025) (width 0.2) (layer "B.Cu") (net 8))
 (segment (start 46.842944 78.7) (end 47.837056 78.7) (width 0.2) (layer "B.Cu") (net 8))
 (segment (start 24.235669 46.12025) (end 23.562015 46.793904) (width 0.2) (layer "B.Cu") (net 8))
 (segment (start 74.55 44.8) (end 73.25 43.5) (width 0.2) (layer "B.Cu") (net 8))
 (segment (start 24.712015 47.27025) (end 24.712015 53.777701) (width 0.2) (layer "B.Cu") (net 9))
 (segment (start 49.189899 76.36) (end 50.01 75.539899) (width 0.2) (layer "B.Cu") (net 9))
 (segment (start 24.712015 53.777701) (end 46.474213 75.539899) (width 0.2) (layer "B.Cu") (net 9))
 (segment (start 50.01 71.74) (end 73.25 48.5) (width 0.2) (layer "B.Cu") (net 9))
 (segment (start 48.030101 76.36) (end 49.189899 76.36) (width 0.2) (layer "B.Cu") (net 9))
 (segment (start 50.01 75.539899) (end 50.01 71.74) (width 0.2) (layer "B.Cu") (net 9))
 (segment (start 46.474213 75.539899) (end 47.21 75.539899) (width 0.2) (layer "B.Cu") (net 9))
 (segment (start 47.21 75.539899) (end 48.030101 76.36) (width 0.2) (layer "B.Cu") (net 9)))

